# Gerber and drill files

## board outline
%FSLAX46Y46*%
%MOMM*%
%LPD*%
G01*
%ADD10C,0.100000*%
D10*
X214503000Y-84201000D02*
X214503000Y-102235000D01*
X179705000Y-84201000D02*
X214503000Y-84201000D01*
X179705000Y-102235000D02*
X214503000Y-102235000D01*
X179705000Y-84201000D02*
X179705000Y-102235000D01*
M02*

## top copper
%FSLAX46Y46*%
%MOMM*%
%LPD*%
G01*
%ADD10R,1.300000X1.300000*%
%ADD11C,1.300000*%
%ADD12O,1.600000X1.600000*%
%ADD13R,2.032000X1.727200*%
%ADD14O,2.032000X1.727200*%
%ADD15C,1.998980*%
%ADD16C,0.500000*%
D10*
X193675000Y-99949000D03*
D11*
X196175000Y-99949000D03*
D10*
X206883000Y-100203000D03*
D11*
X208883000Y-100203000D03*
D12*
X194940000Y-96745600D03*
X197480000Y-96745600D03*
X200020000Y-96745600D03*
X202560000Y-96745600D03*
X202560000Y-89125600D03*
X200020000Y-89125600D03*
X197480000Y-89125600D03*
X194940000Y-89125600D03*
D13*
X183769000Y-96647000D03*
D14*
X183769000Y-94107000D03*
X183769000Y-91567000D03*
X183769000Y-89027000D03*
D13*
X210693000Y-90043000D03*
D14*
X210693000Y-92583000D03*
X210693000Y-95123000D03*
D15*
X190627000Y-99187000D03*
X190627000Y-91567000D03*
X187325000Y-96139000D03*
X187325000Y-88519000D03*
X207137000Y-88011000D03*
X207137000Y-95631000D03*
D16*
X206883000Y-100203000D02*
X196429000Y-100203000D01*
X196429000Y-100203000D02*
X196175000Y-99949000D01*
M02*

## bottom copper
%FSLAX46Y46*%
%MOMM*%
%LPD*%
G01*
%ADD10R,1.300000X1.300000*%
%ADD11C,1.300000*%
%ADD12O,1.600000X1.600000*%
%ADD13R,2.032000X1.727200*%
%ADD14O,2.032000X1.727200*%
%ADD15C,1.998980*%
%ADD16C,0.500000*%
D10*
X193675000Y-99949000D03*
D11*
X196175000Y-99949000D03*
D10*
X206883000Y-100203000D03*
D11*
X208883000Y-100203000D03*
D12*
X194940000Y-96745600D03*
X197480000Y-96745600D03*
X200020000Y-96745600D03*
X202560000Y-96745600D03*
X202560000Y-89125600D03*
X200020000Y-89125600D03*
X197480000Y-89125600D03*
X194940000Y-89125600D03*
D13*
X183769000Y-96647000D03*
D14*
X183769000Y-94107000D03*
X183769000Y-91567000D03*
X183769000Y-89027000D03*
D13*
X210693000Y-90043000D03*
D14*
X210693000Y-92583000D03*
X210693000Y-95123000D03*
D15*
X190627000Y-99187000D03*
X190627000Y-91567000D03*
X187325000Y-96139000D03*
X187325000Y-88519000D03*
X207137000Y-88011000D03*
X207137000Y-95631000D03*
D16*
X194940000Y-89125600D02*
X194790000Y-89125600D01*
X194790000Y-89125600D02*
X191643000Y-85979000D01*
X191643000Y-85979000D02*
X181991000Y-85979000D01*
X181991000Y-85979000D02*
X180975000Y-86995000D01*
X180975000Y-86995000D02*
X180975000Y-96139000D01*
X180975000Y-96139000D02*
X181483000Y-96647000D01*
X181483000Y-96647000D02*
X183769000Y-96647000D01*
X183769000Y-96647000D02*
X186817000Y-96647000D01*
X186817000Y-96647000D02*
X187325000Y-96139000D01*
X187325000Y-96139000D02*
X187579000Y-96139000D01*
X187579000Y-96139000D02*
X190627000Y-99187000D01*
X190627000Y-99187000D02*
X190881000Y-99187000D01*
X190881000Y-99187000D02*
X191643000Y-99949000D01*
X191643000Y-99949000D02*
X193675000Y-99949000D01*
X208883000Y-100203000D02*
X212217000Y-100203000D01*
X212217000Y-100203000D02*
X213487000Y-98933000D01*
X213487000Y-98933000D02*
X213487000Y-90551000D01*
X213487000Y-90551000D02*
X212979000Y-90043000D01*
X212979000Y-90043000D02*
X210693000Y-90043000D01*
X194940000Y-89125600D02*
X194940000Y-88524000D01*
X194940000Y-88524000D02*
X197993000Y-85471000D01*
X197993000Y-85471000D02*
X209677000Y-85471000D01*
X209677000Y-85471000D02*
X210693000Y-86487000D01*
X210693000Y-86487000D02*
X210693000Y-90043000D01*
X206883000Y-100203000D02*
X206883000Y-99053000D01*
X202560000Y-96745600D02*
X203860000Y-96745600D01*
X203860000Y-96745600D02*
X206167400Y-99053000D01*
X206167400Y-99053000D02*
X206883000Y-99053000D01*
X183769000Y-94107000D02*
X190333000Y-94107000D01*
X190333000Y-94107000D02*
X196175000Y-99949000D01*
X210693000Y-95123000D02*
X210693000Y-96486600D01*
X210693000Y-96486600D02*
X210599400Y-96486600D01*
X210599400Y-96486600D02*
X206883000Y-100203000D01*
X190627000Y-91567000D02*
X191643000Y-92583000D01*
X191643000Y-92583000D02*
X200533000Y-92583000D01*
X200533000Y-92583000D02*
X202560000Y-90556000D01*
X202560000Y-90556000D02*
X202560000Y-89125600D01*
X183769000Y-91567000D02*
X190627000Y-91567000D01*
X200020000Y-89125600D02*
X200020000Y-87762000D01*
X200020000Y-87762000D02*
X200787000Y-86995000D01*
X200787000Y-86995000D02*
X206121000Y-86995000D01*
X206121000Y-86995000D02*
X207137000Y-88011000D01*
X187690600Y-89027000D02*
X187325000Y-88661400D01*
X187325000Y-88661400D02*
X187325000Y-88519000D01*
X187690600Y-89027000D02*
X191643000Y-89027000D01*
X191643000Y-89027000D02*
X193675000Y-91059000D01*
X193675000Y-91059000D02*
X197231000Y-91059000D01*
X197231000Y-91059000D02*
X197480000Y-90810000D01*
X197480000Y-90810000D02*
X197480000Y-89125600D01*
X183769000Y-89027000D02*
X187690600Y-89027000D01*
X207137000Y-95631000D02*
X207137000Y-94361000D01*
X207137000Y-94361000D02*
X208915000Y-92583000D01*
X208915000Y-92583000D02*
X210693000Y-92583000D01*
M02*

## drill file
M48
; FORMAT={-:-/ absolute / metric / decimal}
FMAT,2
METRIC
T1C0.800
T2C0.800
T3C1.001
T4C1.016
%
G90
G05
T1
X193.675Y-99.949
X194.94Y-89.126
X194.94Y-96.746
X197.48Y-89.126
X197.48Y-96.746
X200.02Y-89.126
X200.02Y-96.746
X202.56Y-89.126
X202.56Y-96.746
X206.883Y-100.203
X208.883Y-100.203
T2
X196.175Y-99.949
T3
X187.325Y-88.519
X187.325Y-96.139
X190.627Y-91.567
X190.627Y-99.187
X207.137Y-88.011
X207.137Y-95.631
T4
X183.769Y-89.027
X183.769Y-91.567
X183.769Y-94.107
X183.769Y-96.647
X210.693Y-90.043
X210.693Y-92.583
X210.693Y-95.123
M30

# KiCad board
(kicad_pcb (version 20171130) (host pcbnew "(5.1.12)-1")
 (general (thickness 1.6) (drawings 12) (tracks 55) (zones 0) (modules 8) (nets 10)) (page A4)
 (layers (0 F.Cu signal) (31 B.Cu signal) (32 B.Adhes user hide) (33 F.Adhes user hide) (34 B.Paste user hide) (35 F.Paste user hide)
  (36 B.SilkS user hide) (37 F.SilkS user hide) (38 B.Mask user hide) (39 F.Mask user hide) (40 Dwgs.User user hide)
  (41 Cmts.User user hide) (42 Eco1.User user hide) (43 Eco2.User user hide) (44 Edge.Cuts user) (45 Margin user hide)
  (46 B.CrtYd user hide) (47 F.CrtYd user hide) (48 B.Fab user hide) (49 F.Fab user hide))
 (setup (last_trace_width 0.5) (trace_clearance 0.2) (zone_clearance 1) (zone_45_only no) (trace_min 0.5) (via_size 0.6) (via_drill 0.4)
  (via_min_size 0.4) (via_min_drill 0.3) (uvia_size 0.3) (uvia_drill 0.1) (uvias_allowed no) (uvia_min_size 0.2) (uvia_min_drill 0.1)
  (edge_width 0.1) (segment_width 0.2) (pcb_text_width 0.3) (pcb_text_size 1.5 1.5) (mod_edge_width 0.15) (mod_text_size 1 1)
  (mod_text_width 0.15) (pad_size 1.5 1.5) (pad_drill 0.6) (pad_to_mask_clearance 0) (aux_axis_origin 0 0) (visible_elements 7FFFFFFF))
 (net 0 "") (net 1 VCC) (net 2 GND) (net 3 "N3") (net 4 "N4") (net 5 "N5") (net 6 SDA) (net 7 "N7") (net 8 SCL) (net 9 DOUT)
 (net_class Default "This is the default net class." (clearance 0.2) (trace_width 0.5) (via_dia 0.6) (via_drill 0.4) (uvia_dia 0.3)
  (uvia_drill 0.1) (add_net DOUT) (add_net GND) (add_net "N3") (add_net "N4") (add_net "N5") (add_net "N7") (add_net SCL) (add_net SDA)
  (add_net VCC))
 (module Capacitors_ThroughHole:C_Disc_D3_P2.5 (layer F.Cu) (at 193.675 99.949)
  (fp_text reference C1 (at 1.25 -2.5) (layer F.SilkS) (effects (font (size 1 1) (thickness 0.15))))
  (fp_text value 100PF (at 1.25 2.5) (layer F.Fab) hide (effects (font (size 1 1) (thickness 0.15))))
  (pad 1 thru_hole rect (at 0 0) (size 1.3 1.3) (drill 0.8) (layers *.Cu *.Mask F.SilkS) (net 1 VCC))
  (pad 2 thru_hole circle (at 2.5 0) (size 1.3 1.3) (drill 0.8001) (layers *.Cu *.Mask F.SilkS) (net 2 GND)))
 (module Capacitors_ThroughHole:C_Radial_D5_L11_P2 (layer F.Cu) (at 206.883 100.203)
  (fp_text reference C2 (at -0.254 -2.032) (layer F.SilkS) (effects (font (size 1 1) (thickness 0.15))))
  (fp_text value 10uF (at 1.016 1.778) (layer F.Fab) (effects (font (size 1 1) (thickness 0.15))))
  (pad 1 thru_hole rect (at 0 0) (size 1.3 1.3) (drill 0.8) (layers *.Cu *.Mask F.SilkS) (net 2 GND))
  (pad 2 thru_hole circle (at 2 0) (size 1.3 1.3) (drill 0.8) (layers *.Cu *.Mask F.SilkS) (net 1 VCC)))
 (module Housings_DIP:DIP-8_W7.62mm (layer F.Cu) (at 194.94 96.7456 90)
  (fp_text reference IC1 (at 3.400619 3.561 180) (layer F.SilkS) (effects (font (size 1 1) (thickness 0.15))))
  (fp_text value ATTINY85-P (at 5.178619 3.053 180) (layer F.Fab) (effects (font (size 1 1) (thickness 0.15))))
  (pad 1 thru_hole oval (at 0 0 90) (size 1.6 1.6) (drill 0.8) (layers *.Cu *.Mask F.SilkS) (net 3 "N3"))
  (pad 2 thru_hole oval (at 0 2.54 90) (size 1.6 1.6) (drill 0.8) (layers *.Cu *.Mask F.SilkS) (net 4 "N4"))
  (pad 3 thru_hole oval (at 0 5.08 90) (size 1.6 1.6) (drill 0.8) (layers *.Cu *.Mask F.SilkS) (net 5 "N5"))
  (pad 4 thru_hole oval (at 0 7.62 90) (size 1.6 1.6) (drill 0.8) (layers *.Cu *.Mask F.SilkS) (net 2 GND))
  (pad 5 thru_hole oval (at 7.62 7.62 90) (size 1.6 1.6) (drill 0.8) (layers *.Cu *.Mask F.SilkS) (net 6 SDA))
  (pad 6 thru_hole oval (at 7.62 5.08 90) (size 1.6 1.6) (drill 0.8) (layers *.Cu *.Mask F.SilkS) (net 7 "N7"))
  (pad 7 thru_hole oval (at 7.62 2.54 90) (size 1.6 1.6) (drill 0.8) (layers *.Cu *.Mask F.SilkS) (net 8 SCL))
  (pad 8 thru_hole oval (at 7.62 0 90) (size 1.6 1.6) (drill 0.8) (layers *.Cu *.Mask F.SilkS) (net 1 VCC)))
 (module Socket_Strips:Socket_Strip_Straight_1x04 (layer F.Cu) (at 183.769 96.647 90)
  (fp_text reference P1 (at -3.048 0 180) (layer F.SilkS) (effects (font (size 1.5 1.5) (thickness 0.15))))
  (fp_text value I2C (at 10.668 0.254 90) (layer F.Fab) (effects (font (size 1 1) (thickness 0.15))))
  (pad 1 thru_hole rect (at 0 0 90) (size 1.7272 2.032) (drill 1.016) (layers *.Cu *.Mask F.SilkS) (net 1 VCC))
  (pad 2 thru_hole oval (at 2.54 0 90) (size 1.7272 2.032) (drill 1.016) (layers *.Cu *.Mask F.SilkS) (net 2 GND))
  (pad 3 thru_hole oval (at 5.08 0 90) (size 1.7272 2.032) (drill 1.016) (layers *.Cu *.Mask F.SilkS) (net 6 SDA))
  (pad 4 thru_hole oval (at 7.62 0 90) (size 1.7272 2.032) (drill 1.016) (layers *.Cu *.Mask F.SilkS) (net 8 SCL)))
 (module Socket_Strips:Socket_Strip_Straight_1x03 (layer F.Cu) (at 210.693 90.043 270)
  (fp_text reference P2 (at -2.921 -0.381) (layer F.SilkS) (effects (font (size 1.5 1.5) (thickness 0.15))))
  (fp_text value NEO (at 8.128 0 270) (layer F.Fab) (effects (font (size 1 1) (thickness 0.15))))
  (pad 1 thru_hole rect (at 0 0 270) (size 1.7272 2.032) (drill 1.016) (layers *.Cu *.Mask F.SilkS) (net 1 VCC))
  (pad 2 thru_hole oval (at 2.54 0 270) (size 1.7272 2.032) (drill 1.016) (layers *.Cu *.Mask F.SilkS) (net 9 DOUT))
  (pad 3 thru_hole oval (at 5.08 0 270) (size 1.7272 2.032) (drill 1.016) (layers *.Cu *.Mask F.SilkS) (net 2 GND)))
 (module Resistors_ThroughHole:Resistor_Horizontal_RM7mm (layer F.Cu) (at 190.627 99.187 90)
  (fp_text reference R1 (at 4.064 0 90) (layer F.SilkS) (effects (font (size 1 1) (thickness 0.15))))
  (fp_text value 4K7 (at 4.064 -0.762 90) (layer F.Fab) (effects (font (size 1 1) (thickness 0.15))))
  (pad 1 thru_hole circle (at 0 0 90) (size 1.99898 1.99898) (drill 1.00076) (layers *.Cu *.SilkS *.Mask) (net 1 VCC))
  (pad 2 thru_hole circle (at 7.62 0 90) (size 1.99898 1.99898) (drill 1.00076) (layers *.Cu *.SilkS *.Mask) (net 6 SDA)))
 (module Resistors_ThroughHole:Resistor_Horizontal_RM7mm (layer F.Cu) (at 187.325 96.139 90)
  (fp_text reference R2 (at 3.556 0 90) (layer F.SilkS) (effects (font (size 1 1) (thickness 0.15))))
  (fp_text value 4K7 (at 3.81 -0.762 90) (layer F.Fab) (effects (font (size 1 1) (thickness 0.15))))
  (pad 1 thru_hole circle (at 0 0 90) (size 1.99898 1.99898) (drill 1.00076) (layers *.Cu *.SilkS *.Mask) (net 1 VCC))
  (pad 2 thru_hole circle (at 7.62 0 90) (size 1.99898 1.99898) (drill 1.00076) (layers *.Cu *.SilkS *.Mask) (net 8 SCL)))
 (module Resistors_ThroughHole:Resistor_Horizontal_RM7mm (layer F.Cu) (at 207.137 88.011 270)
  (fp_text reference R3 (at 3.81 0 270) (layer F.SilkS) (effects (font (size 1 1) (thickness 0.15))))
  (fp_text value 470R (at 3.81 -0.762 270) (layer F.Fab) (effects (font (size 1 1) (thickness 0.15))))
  (pad 1 thru_hole circle (at 0 0 270) (size 1.99898 1.99898) (drill 1.00076) (layers *.Cu *.SilkS *.Mask) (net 7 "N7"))
  (pad 2 thru_hole circle (at 7.62 0 270) (size 1.99898 1.99898) (drill 1.00076) (layers *.Cu *.SilkS *.Mask) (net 9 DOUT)))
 (gr_line (start 214.503 84.201) (end 214.503 102.235) (angle 90) (layer Edge.Cuts) (width 0.1))
 (gr_line (start 179.705 84.201) (end 214.503 84.201) (angle 90) (layer Edge.Cuts) (width 0.1))
 (gr_line (start 179.705 102.235) (end 214.503 102.235) (angle 90) (layer Edge.Cuts) (width 0.1))
 (gr_line (start 179.705 84.201) (end 179.705 102.235) (angle 90) (layer Edge.Cuts) (width 0.1))
 (segment (start 194.94 89.1256) (end 194.79 89.1256) (width 0.5) (layer B.Cu) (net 1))
 (segment (start 194.79 89.1256) (end 191.643 85.979) (width 0.5) (layer B.Cu) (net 1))
 (segment (start 191.643 85.979) (end 181.991 85.979) (width 0.5) (layer B.Cu) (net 1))
 (segment (start 181.991 85.979) (end 180.975 86.995) (width 0.5) (layer B.Cu) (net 1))
 (segment (start 180.975 86.995) (end 180.975 96.139) (width 0.5) (layer B.Cu) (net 1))
 (segment (start 180.975 96.139) (end 181.483 96.647) (width 0.5) (layer B.Cu) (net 1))
 (segment (start 181.483 96.647) (end 183.769 96.647) (width 0.5) (layer B.Cu) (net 1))
 (segment (start 183.769 96.647) (end 186.817 96.647) (width 0.5) (layer B.Cu) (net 1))
 (segment (start 186.817 96.647) (end 187.325 96.139) (width 0.5) (layer B.Cu) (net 1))
 (segment (start 187.325 96.139) (end 187.579 96.139) (width 0.5) (layer B.Cu) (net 1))
 (segment (start 187.579 96.139) (end 190.627 99.187) (width 0.5) (layer B.Cu) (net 1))
 (segment (start 190.627 99.187) (end 190.881 99.187) (width 0.5) (layer B.Cu) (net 1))
 (segment (start 190.881 99.187) (end 191.643 99.949) (width 0.5) (layer B.Cu) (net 1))
 (segment (start 191.643 99.949) (end 193.675 99.949) (width 0.5) (layer B.Cu) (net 1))
 (segment (start 208.883 100.203) (end 212.217 100.203) (width 0.5) (layer B.Cu) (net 1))
 (segment (start 212.217 100.203) (end 213.487 98.933) (width 0.5) (layer B.Cu) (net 1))
 (segment (start 213.487 98.933) (end 213.487 90.551) (width 0.5) (layer B.Cu) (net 1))
 (segment (start 213.487 90.551) (end 212.979 90.043) (width 0.5) (layer B.Cu) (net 1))
 (segment (start 212.979 90.043) (end 210.693 90.043) (width 0.5) (layer B.Cu) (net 1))
 (segment (start 194.94 89.1256) (end 194.94 88.524) (width 0.5) (layer B.Cu) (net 1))
 (segment (start 194.94 88.524) (end 197.993 85.471) (width 0.5) (layer B.Cu) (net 1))
 (segment (start 197.993 85.471) (end 209.677 85.471) (width 0.5) (layer B.Cu) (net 1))
 (segment (start 209.677 85.471) (end 210.693 86.487) (width 0.5) (layer B.Cu) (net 1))
 (segment (start 210.693 86.487) (end 210.693 90.043) (width 0.5) (layer B.Cu) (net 1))
 (segment (start 206.883 100.203) (end 196.429 100.203) (width 0.5) (layer F.Cu) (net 2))
 (segment (start 196.429 100.203) (end 196.175 99.949) (width 0.5) (layer F.Cu) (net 2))
 (segment (start 206.883 100.203) (end 206.883 99.053) (width 0.5) (layer B.Cu) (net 2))
 (segment (start 202.56 96.7456) (end 203.86 96.7456) (width 0.5) (layer B.Cu) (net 2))
 (segment (start 203.86 96.7456) (end 206.1674 99.053) (width 0.5) (layer B.Cu) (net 2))
 (segment (start 206.1674 99.053) (end 206.883 99.053) (width 0.5) (layer B.Cu) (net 2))
 (segment (start 183.769 94.107) (end 190.333 94.107) (width 0.5) (layer B.Cu) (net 2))
 (segment (start 190.333 94.107) (end 196.175 99.949) (width 0.5) (layer B.Cu) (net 2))
 (segment (start 210.693 95.123) (end 210.693 96.4866) (width 0.5) (layer B.Cu) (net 2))
 (segment (start 210.693 96.4866) (end 210.5994 96.4866) (width 0.5) (layer B.Cu) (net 2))
 (segment (start 210.5994 96.4866) (end 206.883 100.203) (width 0.5) (layer B.Cu) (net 2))
 (segment (start 190.627 91.567) (end 191.643 92.583) (width 0.5) (layer B.Cu) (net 6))
 (segment (start 191.643 92.583) (end 200.533 92.583) (width 0.5) (layer B.Cu) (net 6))
 (segment (start 200.533 92.583) (end 202.56 90.556) (width 0.5) (layer B.Cu) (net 6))
 (segment (start 202.56 90.556) (end 202.56 89.1256) (width 0.5) (layer B.Cu) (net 6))
 (segment (start 183.769 91.567) (end 190.627 91.567) (width 0.5) (layer B.Cu) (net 6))
 (segment (start 200.02 89.1256) (end 200.02 87.762) (width 0.5) (layer B.Cu) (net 7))
 (segment (start 200.02 87.762) (end 200.787 86.995) (width 0.5) (layer B.Cu) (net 7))
 (segment (start 200.787 86.995) (end 206.121 86.995) (width 0.5) (layer B.Cu) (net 7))
 (segment (start 206.121 86.995) (end 207.137 88.011) (width 0.5) (layer B.Cu) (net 7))
 (segment (start 187.6906 89.027) (end 187.325 88.6614) (width 0.5) (layer B.Cu) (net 8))
 (segment (start 187.325 88.6614) (end 187.325 88.519) (width 0.5) (layer B.Cu) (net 8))
 (segment (start 187.6906 89.027) (end 191.643 89.027) (width 0.5) (layer B.Cu) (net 8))
 (segment (start 191.643 89.027) (end 193.675 91.059) (width 0.5) (layer B.Cu) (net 8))
 (segment (start 193.675 91.059) (end 197.231 91.059) (width 0.5) (layer B.Cu) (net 8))
 (segment (start 197.231 91.059) (end 197.48 90.81) (width 0.5) (layer B.Cu) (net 8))
 (segment (start 197.48 90.81) (end 197.48 89.1256) (width 0.5) (layer B.Cu) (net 8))
 (segment (start 183.769 89.027) (end 187.6906 89.027) (width 0.5) (layer B.Cu) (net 8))
 (segment (start 207.137 95.631) (end 207.137 94.361) (width 0.5) (layer B.Cu) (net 9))
 (segment (start 207.137 94.361) (end 208.915 92.583) (width 0.5) (layer B.Cu) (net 9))
 (segment (start 208.915 92.583) (end 210.693 92.583) (width 0.5) (layer B.Cu) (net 9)))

